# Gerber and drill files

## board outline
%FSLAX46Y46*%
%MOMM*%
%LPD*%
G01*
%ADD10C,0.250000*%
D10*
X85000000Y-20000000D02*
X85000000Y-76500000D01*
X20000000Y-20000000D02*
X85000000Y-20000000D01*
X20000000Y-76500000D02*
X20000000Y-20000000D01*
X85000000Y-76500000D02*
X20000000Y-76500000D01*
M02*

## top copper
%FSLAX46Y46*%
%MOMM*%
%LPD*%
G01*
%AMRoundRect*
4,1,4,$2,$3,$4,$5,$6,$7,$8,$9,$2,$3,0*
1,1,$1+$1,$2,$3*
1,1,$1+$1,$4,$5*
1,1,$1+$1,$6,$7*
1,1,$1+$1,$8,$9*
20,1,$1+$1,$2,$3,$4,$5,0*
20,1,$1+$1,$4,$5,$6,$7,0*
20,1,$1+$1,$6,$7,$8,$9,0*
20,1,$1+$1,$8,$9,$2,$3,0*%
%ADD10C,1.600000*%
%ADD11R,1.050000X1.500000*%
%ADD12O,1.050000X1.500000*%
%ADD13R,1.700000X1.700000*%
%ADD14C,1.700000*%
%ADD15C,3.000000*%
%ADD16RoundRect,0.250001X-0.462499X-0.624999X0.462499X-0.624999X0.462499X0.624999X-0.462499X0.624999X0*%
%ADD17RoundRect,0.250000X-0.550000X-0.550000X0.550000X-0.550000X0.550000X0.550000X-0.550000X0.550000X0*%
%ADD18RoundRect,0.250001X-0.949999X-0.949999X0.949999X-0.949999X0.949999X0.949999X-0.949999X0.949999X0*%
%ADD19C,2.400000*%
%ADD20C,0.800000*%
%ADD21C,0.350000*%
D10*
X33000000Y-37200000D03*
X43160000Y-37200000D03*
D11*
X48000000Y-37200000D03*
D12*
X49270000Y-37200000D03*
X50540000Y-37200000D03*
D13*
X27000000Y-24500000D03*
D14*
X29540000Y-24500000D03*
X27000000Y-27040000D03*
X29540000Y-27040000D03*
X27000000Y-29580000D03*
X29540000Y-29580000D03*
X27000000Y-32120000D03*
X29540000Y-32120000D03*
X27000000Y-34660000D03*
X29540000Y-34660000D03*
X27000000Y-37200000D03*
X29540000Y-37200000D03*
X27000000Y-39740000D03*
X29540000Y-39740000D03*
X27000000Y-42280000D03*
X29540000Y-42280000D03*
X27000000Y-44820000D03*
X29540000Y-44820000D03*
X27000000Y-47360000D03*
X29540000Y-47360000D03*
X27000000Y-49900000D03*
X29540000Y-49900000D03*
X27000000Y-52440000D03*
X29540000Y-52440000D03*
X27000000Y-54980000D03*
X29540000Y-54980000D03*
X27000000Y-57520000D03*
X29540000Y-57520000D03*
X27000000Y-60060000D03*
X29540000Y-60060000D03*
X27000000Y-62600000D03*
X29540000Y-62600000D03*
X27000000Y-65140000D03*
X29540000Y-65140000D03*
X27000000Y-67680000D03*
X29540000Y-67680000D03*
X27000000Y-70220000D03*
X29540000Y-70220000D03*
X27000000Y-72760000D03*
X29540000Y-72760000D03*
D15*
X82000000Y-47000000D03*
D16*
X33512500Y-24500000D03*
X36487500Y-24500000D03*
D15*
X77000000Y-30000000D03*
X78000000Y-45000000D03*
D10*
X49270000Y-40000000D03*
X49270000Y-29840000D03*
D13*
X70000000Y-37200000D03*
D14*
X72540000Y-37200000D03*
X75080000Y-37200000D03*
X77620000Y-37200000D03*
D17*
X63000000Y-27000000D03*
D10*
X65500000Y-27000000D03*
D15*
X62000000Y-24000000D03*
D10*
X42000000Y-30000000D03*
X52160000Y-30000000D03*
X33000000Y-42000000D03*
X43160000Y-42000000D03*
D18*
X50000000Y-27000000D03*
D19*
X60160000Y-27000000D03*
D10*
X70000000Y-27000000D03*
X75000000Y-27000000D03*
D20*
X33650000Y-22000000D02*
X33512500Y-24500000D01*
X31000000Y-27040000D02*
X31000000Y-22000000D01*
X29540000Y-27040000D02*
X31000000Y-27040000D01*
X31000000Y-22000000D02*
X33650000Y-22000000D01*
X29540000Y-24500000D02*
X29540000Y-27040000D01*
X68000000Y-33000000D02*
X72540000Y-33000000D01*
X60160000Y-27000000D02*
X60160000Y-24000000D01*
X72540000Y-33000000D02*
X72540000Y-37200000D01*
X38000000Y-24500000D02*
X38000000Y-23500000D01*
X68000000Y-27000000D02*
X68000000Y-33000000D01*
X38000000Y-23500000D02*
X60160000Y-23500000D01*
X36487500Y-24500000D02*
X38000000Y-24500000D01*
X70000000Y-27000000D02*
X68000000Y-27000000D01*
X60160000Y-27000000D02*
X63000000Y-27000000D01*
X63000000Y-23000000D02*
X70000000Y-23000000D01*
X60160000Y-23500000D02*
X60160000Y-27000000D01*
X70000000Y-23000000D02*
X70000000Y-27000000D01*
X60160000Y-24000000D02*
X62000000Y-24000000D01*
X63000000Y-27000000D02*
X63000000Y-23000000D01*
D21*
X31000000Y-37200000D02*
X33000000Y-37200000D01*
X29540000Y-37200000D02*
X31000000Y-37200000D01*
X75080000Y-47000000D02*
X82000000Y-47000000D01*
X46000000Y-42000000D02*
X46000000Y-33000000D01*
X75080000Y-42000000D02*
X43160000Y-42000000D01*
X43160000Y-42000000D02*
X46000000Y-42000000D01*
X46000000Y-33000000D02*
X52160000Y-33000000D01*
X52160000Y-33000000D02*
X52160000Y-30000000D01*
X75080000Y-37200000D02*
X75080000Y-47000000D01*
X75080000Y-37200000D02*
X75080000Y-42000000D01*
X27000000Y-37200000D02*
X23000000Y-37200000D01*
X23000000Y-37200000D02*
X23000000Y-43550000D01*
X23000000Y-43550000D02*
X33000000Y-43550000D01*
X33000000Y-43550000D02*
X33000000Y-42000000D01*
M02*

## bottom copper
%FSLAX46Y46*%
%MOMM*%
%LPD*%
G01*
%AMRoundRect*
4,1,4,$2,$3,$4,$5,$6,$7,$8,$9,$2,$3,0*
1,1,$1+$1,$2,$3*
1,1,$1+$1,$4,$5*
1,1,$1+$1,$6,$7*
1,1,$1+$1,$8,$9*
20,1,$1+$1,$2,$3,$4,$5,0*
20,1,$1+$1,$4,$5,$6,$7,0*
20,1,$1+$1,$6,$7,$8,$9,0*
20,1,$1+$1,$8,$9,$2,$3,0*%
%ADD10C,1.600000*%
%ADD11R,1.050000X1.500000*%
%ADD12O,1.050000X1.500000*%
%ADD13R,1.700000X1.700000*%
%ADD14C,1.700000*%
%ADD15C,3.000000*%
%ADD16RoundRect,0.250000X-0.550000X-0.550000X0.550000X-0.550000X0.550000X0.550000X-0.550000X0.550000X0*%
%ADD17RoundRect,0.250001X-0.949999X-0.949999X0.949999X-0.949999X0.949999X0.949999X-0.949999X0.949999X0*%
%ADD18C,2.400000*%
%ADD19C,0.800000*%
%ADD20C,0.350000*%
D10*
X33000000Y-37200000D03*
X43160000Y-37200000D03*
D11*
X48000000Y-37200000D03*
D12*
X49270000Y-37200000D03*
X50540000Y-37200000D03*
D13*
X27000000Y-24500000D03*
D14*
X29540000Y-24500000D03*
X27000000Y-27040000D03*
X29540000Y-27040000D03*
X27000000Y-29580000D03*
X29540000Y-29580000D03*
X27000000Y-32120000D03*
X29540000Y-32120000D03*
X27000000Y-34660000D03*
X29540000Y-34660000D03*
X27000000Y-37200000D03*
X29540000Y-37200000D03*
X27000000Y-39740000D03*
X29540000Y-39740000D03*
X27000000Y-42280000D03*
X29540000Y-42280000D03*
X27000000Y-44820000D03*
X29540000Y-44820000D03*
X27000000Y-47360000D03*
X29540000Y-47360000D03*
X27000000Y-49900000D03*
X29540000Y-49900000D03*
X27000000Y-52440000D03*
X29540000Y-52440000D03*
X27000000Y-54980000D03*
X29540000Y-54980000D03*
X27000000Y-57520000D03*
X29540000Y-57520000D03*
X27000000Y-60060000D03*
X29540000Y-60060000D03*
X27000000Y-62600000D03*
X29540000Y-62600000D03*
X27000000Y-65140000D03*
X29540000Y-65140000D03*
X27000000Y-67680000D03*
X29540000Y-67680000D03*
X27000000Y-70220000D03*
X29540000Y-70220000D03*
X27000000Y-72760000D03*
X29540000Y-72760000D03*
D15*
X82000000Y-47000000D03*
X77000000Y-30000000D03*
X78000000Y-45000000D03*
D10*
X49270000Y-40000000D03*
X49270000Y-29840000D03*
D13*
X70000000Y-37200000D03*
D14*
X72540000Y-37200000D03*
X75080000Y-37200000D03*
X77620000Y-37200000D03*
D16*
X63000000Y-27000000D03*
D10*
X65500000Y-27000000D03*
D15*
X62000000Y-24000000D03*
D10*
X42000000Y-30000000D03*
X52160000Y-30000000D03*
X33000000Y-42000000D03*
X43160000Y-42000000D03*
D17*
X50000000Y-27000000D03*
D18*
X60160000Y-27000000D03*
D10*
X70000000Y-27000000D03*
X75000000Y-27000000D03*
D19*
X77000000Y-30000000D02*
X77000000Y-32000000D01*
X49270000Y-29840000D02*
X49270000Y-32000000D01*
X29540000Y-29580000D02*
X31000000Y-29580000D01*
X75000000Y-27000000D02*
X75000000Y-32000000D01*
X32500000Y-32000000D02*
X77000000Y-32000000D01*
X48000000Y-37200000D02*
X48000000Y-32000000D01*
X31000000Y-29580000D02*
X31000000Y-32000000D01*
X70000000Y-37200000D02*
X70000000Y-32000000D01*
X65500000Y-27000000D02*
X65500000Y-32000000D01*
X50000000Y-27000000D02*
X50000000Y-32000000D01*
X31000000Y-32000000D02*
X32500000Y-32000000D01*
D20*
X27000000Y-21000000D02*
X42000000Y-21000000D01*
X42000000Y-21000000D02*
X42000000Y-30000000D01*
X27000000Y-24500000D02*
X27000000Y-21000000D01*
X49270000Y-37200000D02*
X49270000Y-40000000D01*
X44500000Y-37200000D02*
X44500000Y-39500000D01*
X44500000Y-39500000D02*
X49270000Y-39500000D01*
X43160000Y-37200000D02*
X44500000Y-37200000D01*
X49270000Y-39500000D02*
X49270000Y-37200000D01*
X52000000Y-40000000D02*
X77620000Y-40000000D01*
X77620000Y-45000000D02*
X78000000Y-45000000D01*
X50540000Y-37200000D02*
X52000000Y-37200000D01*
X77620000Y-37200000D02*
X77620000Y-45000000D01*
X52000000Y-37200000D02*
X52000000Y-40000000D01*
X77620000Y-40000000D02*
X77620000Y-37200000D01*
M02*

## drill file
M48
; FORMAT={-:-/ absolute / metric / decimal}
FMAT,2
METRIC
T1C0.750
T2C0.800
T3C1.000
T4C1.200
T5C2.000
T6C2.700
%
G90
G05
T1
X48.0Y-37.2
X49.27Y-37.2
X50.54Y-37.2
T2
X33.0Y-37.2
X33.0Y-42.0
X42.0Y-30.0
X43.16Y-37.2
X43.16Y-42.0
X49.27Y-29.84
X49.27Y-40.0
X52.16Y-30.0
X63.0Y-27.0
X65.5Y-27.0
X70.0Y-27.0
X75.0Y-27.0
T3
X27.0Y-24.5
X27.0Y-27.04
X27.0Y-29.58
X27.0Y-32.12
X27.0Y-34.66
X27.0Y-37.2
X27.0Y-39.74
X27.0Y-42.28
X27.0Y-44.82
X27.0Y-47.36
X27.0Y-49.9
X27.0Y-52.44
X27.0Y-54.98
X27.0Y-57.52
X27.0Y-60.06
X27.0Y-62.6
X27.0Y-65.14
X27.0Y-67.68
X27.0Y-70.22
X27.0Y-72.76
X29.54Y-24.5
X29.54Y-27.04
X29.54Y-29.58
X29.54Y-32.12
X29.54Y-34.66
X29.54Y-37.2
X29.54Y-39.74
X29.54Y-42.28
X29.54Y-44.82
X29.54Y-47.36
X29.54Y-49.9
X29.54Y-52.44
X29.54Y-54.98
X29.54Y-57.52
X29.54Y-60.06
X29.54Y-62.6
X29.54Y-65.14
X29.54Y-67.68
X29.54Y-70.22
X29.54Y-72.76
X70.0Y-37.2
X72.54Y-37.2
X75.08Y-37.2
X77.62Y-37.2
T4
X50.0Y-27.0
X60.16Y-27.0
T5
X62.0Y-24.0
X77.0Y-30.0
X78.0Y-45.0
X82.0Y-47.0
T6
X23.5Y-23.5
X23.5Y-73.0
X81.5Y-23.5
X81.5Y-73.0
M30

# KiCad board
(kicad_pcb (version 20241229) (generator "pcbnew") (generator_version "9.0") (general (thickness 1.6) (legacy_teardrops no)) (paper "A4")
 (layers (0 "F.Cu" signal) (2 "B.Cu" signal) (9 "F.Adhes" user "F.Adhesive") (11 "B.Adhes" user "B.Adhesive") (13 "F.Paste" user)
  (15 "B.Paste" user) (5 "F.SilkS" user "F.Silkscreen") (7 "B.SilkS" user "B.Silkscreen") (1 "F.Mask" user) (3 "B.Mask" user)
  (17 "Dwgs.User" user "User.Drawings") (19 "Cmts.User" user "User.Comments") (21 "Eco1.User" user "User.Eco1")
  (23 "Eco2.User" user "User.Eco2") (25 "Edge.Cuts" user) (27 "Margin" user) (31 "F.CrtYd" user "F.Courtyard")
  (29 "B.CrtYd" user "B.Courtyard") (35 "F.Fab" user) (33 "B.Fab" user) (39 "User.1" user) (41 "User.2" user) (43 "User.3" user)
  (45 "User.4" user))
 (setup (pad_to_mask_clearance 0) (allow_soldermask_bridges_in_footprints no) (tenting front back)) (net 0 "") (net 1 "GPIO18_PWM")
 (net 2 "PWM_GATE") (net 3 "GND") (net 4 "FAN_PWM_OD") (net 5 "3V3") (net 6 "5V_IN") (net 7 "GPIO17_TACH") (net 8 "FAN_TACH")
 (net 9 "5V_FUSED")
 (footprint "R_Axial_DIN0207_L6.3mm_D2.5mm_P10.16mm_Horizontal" (layer "F.Cu") (at 33 37.2)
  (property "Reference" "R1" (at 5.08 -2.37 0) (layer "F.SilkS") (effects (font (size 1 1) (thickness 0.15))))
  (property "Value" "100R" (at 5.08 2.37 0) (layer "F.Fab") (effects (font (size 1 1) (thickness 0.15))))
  (pad "1" thru_hole circle (at 0 0) (size 1.6 1.6) (drill 0.8) (layers "*.Cu" "*.Mask") (remove_unused_layers no) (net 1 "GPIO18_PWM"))
  (pad "2" thru_hole circle (at 10.16 0) (size 1.6 1.6) (drill 0.8) (layers "*.Cu" "*.Mask") (remove_unused_layers no) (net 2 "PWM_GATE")))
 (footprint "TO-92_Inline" (layer "F.Cu") (at 48 37.2)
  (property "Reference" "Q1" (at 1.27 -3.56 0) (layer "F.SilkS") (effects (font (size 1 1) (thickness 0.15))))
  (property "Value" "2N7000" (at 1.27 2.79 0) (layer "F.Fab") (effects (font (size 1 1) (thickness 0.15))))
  (pad "1" thru_hole rect (at 0 0) (size 1.05 1.5) (drill 0.75) (layers "*.Cu" "*.Mask") (remove_unused_layers no) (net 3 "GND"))
  (pad "2" thru_hole oval (at 1.27 0) (size 1.05 1.5) (drill 0.75) (layers "*.Cu" "*.Mask") (remove_unused_layers no) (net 2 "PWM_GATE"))
  (pad "3" thru_hole oval (at 2.54 0) (size 1.05 1.5) (drill 0.75) (layers "*.Cu" "*.Mask") (remove_unused_layers no) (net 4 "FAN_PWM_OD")))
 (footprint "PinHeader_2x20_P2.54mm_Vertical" (layer "F.Cu") (at 27 24.5)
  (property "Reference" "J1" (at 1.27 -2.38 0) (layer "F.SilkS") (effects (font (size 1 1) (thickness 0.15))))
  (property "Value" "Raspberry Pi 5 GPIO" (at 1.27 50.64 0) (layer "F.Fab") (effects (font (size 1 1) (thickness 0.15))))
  (pad "1" thru_hole rect (at 0 0) (size 1.7 1.7) (drill 1) (layers "*.Cu" "*.Mask") (remove_unused_layers no) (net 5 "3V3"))
  (pad "2" thru_hole circle (at 2.54 0) (size 1.7 1.7) (drill 1) (layers "*.Cu" "*.Mask") (remove_unused_layers no) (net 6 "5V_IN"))
  (pad "3" thru_hole circle (at 0 2.54) (size 1.7 1.7) (drill 1) (layers "*.Cu" "*.Mask") (remove_unused_layers no))
  (pad "4" thru_hole circle (at 2.54 2.54) (size 1.7 1.7) (drill 1) (layers "*.Cu" "*.Mask") (remove_unused_layers no) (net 6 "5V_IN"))
  (pad "5" thru_hole circle (at 0 5.08) (size 1.7 1.7) (drill 1) (layers "*.Cu" "*.Mask") (remove_unused_layers no))
  (pad "6" thru_hole circle (at 2.54 5.08) (size 1.7 1.7) (drill 1) (layers "*.Cu" "*.Mask") (remove_unused_layers no) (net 3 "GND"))
  (pad "7" thru_hole circle (at 0 7.62) (size 1.7 1.7) (drill 1) (layers "*.Cu" "*.Mask") (remove_unused_layers no))
  (pad "8" thru_hole circle (at 2.54 7.62) (size 1.7 1.7) (drill 1) (layers "*.Cu" "*.Mask") (remove_unused_layers no))
  (pad "9" thru_hole circle (at 0 10.16) (size 1.7 1.7) (drill 1) (layers "*.Cu" "*.Mask") (remove_unused_layers no))
  (pad "10" thru_hole circle (at 2.54 10.16) (size 1.7 1.7) (drill 1) (layers "*.Cu" "*.Mask") (remove_unused_layers no))
  (pad "11" thru_hole circle (at 0 12.7) (size 1.7 1.7) (drill 1) (layers "*.Cu" "*.Mask") (remove_unused_layers no) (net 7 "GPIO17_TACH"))
  (pad "12" thru_hole circle (at 2.54 12.7) (size 1.7 1.7) (drill 1) (layers "*.Cu" "*.Mask") (remove_unused_layers no) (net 1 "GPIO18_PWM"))
  (pad "13" thru_hole circle (at 0 15.24) (size 1.7 1.7) (drill 1) (layers "*.Cu" "*.Mask") (remove_unused_layers no))
  (pad "14" thru_hole circle (at 2.54 15.24) (size 1.7 1.7) (drill 1) (layers "*.Cu" "*.Mask") (remove_unused_layers no))
  (pad "15" thru_hole circle (at 0 17.78) (size 1.7 1.7) (drill 1) (layers "*.Cu" "*.Mask") (remove_unused_layers no))
  (pad "16" thru_hole circle (at 2.54 17.78) (size 1.7 1.7) (drill 1) (layers "*.Cu" "*.Mask") (remove_unused_layers no))
  (pad "17" thru_hole circle (at 0 20.32) (size 1.7 1.7) (drill 1) (layers "*.Cu" "*.Mask") (remove_unused_layers no))
  (pad "18" thru_hole circle (at 2.54 20.32) (size 1.7 1.7) (drill 1) (layers "*.Cu" "*.Mask") (remove_unused_layers no))
  (pad "19" thru_hole circle (at 0 22.86) (size 1.7 1.7) (drill 1) (layers "*.Cu" "*.Mask") (remove_unused_layers no))
  (pad "20" thru_hole circle (at 2.54 22.86) (size 1.7 1.7) (drill 1) (layers "*.Cu" "*.Mask") (remove_unused_layers no))
  (pad "21" thru_hole circle (at 0 25.4) (size 1.7 1.7) (drill 1) (layers "*.Cu" "*.Mask") (remove_unused_layers no))
  (pad "22" thru_hole circle (at 2.54 25.4) (size 1.7 1.7) (drill 1) (layers "*.Cu" "*.Mask") (remove_unused_layers no))
  (pad "23" thru_hole circle (at 0 27.94) (size 1.7 1.7) (drill 1) (layers "*.Cu" "*.Mask") (remove_unused_layers no))
  (pad "24" thru_hole circle (at 2.54 27.94) (size 1.7 1.7) (drill 1) (layers "*.Cu" "*.Mask") (remove_unused_layers no))
  (pad "25" thru_hole circle (at 0 30.48) (size 1.7 1.7) (drill 1) (layers "*.Cu" "*.Mask") (remove_unused_layers no))
  (pad "26" thru_hole circle (at 2.54 30.48) (size 1.7 1.7) (drill 1) (layers "*.Cu" "*.Mask") (remove_unused_layers no))
  (pad "27" thru_hole circle (at 0 33.02) (size 1.7 1.7) (drill 1) (layers "*.Cu" "*.Mask") (remove_unused_layers no))
  (pad "28" thru_hole circle (at 2.54 33.02) (size 1.7 1.7) (drill 1) (layers "*.Cu" "*.Mask") (remove_unused_layers no))
  (pad "29" thru_hole circle (at 0 35.56) (size 1.7 1.7) (drill 1) (layers "*.Cu" "*.Mask") (remove_unused_layers no))
  (pad "30" thru_hole circle (at 2.54 35.56) (size 1.7 1.7) (drill 1) (layers "*.Cu" "*.Mask") (remove_unused_layers no))
  (pad "31" thru_hole circle (at 0 38.1) (size 1.7 1.7) (drill 1) (layers "*.Cu" "*.Mask") (remove_unused_layers no))
  (pad "32" thru_hole circle (at 2.54 38.1) (size 1.7 1.7) (drill 1) (layers "*.Cu" "*.Mask") (remove_unused_layers no))
  (pad "33" thru_hole circle (at 0 40.64) (size 1.7 1.7) (drill 1) (layers "*.Cu" "*.Mask") (remove_unused_layers no))
  (pad "34" thru_hole circle (at 2.54 40.64) (size 1.7 1.7) (drill 1) (layers "*.Cu" "*.Mask") (remove_unused_layers no))
  (pad "35" thru_hole circle (at 0 43.18) (size 1.7 1.7) (drill 1) (layers "*.Cu" "*.Mask") (remove_unused_layers no))
  (pad "36" thru_hole circle (at 2.54 43.18) (size 1.7 1.7) (drill 1) (layers "*.Cu" "*.Mask") (remove_unused_layers no))
  (pad "37" thru_hole circle (at 0 45.72) (size 1.7 1.7) (drill 1) (layers "*.Cu" "*.Mask") (remove_unused_layers no))
  (pad "38" thru_hole circle (at 2.54 45.72) (size 1.7 1.7) (drill 1) (layers "*.Cu" "*.Mask") (remove_unused_layers no))
  (pad "39" thru_hole circle (at 0 48.26) (size 1.7 1.7) (drill 1) (layers "*.Cu" "*.Mask") (remove_unused_layers no))
  (pad "40" thru_hole circle (at 2.54 48.26) (size 1.7 1.7) (drill 1) (layers "*.Cu" "*.Mask") (remove_unused_layers no)))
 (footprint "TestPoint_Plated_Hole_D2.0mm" (layer "F.Cu") (at 82 47)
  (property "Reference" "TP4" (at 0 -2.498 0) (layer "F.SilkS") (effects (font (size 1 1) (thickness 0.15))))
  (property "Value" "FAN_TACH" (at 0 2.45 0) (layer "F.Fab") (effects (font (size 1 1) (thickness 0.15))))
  (pad "1" thru_hole circle (at 0 0) (size 3 3) (drill 2) (layers "*.Cu" "*.Mask") (remove_unused_layers no) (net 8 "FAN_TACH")))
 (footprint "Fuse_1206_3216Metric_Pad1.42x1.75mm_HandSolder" (layer "F.Cu") (at 35 24.5)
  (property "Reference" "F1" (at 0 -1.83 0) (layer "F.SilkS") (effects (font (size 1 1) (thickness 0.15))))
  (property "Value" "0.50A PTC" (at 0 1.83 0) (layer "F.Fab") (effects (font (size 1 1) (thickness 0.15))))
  (pad "1" smd roundrect (at -1.4875 0) (size 1.425 1.75) (layers "F.Cu" "F.Mask" "F.Paste") (roundrect_rratio 0.175439) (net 6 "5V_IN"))
  (pad "2" smd roundrect (at 1.4875 0) (size 1.425 1.75) (layers "F.Cu" "F.Mask" "F.Paste") (roundrect_rratio 0.175439) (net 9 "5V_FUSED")))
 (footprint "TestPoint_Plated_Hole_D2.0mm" (layer "F.Cu") (at 77 30)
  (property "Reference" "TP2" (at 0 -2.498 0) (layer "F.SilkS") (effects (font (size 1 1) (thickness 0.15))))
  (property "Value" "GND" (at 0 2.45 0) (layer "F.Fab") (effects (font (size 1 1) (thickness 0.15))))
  (pad "1" thru_hole circle (at 0 0) (size 3 3) (drill 2) (layers "*.Cu" "*.Mask") (remove_unused_layers no) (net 3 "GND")))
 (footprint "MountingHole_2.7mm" (layer "F.Cu") (at 81.5 23.5)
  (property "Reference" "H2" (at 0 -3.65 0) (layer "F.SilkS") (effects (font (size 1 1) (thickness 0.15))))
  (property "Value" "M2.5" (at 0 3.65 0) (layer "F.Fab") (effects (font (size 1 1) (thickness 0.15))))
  (pad "" np_thru_hole circle (at 0 0) (size 2.7 2.7) (drill 2.7) (layers "*.Cu" "*.Mask")))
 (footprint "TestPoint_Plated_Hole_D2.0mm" (layer "F.Cu") (at 78 45)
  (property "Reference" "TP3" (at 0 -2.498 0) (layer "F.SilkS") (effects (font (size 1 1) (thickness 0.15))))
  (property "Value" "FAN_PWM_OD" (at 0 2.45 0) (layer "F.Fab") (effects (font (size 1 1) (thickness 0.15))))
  (pad "1" thru_hole circle (at 0 0) (size 3 3) (drill 2) (layers "*.Cu" "*.Mask") (remove_unused_layers no) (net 4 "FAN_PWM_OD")))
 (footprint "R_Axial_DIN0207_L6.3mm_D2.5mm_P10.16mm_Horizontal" (layer "F.Cu") (at 49.27 40 90)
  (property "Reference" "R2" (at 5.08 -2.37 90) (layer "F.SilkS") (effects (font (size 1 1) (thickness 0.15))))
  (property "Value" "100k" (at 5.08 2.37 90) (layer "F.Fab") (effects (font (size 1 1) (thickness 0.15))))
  (pad "1" thru_hole circle (at 0 0 90) (size 1.6 1.6) (drill 0.8) (layers "*.Cu" "*.Mask") (remove_unused_layers no) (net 2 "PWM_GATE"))
  (pad "2" thru_hole circle (at 10.16 0 90) (size 1.6 1.6) (drill 0.8) (layers "*.Cu" "*.Mask") (remove_unused_layers no) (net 3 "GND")))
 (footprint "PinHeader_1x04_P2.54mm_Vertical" (layer "F.Cu") (at 70 37.2 90)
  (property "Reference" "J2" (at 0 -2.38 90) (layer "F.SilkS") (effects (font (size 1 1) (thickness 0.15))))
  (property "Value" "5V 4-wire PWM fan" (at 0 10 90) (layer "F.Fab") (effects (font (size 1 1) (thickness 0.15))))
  (pad "1" thru_hole rect (at 0 0 90) (size 1.7 1.7) (drill 1) (layers "*.Cu" "*.Mask") (remove_unused_layers no) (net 3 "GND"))
  (pad "2" thru_hole circle (at 0 2.54 90) (size 1.7 1.7) (drill 1) (layers "*.Cu" "*.Mask") (remove_unused_layers no) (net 9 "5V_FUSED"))
  (pad "3" thru_hole circle (at 0 5.08 90) (size 1.7 1.7) (drill 1) (layers "*.Cu" "*.Mask") (remove_unused_layers no) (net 8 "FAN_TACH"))
  (pad "4" thru_hole circle (at 0 7.62 90) (size 1.7 1.7) (drill 1) (layers "*.Cu" "*.Mask") (remove_unused_layers no) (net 4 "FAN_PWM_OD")))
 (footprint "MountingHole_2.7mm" (layer "F.Cu") (at 81.5 73)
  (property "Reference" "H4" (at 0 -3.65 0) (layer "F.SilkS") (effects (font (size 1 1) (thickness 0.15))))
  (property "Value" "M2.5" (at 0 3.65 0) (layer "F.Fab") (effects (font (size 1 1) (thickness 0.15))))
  (pad "" np_thru_hole circle (at 0 0) (size 2.7 2.7) (drill 2.7) (layers "*.Cu" "*.Mask")))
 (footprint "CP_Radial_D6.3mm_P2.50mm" (layer "F.Cu") (at 63 27)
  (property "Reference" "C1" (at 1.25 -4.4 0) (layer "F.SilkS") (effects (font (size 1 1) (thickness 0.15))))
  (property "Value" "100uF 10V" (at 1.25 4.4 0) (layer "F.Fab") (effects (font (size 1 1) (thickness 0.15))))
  (pad "1" thru_hole roundrect (at 0 0) (size 1.6 1.6) (drill 0.8) (layers "*.Cu" "*.Mask") (remove_unused_layers no)
   (roundrect_rratio 0.15625) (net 9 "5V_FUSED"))
  (pad "2" thru_hole circle (at 2.5 0) (size 1.6 1.6) (drill 0.8) (layers "*.Cu" "*.Mask") (remove_unused_layers no) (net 3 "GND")))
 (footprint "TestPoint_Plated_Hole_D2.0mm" (layer "F.Cu") (at 62 24)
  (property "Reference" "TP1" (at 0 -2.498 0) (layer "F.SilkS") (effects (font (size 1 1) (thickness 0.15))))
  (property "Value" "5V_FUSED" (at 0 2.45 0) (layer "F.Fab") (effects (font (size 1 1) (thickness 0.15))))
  (pad "1" thru_hole circle (at 0 0) (size 3 3) (drill 2) (layers "*.Cu" "*.Mask") (remove_unused_layers no) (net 9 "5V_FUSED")))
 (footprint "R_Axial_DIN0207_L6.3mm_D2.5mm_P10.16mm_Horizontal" (layer "F.Cu") (at 42 30)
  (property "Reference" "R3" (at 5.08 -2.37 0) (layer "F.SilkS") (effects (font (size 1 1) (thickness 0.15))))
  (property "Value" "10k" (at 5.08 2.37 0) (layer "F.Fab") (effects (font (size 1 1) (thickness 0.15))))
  (pad "1" thru_hole circle (at 0 0) (size 1.6 1.6) (drill 0.8) (layers "*.Cu" "*.Mask") (remove_unused_layers no) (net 5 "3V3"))
  (pad "2" thru_hole circle (at 10.16 0) (size 1.6 1.6) (drill 0.8) (layers "*.Cu" "*.Mask") (remove_unused_layers no) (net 8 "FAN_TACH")))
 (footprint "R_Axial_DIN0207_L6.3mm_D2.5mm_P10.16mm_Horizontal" (layer "F.Cu") (at 33 42)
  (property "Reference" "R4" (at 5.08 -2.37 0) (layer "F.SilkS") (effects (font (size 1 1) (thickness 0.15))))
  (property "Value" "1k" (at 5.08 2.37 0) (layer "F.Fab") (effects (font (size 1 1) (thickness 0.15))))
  (pad "1" thru_hole circle (at 0 0) (size 1.6 1.6) (drill 0.8) (layers "*.Cu" "*.Mask") (remove_unused_layers no) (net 7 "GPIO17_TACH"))
  (pad "2" thru_hole circle (at 10.16 0) (size 1.6 1.6) (drill 0.8) (layers "*.Cu" "*.Mask") (remove_unused_layers no) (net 8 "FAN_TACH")))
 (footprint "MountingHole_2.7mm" (layer "F.Cu") (at 23.5 73)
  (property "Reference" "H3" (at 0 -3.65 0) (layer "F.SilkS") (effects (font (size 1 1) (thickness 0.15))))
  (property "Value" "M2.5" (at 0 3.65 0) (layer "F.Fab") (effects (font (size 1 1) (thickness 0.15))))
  (pad "" np_thru_hole circle (at 0 0) (size 2.7 2.7) (drill 2.7) (layers "*.Cu" "*.Mask")))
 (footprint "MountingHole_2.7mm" (layer "F.Cu") (at 23.5 23.5)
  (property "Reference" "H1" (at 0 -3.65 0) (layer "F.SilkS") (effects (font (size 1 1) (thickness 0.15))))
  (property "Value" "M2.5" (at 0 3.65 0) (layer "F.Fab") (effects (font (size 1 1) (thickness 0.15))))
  (pad "" np_thru_hole circle (at 0 0) (size 2.7 2.7) (drill 2.7) (layers "*.Cu" "*.Mask")))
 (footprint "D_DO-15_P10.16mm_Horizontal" (layer "F.Cu") (at 50 27)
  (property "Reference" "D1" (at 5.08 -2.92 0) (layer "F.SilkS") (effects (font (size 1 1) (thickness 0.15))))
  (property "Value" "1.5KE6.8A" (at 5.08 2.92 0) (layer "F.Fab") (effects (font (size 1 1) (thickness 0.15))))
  (pad "1" thru_hole roundrect (at 0 0) (size 2.4 2.4) (drill 1.2) (layers "*.Cu" "*.Mask") (remove_unused_layers no)
   (roundrect_rratio 0.104167) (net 3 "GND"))
  (pad "2" thru_hole circle (at 10.16 0) (size 2.4 2.4) (drill 1.2) (layers "*.Cu" "*.Mask") (remove_unused_layers no) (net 9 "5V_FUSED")))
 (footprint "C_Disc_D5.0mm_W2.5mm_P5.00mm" (layer "F.Cu") (at 70 27)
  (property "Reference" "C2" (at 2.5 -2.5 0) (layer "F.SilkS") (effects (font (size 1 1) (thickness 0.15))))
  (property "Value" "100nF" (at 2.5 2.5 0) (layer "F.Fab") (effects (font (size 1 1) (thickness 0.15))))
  (pad "1" thru_hole circle (at 0 0) (size 1.6 1.6) (drill 0.8) (layers "*.Cu" "*.Mask") (remove_unused_layers no) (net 9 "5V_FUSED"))
  (pad "2" thru_hole circle (at 5 0) (size 1.6 1.6) (drill 0.8) (layers "*.Cu" "*.Mask") (remove_unused_layers no) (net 3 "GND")))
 (gr_line (start 85 20) (end 85 76.5) (stroke (width 0.25) (type default)) (layer "Edge.Cuts"))
 (gr_line (start 20 20) (end 85 20) (stroke (width 0.25) (type default)) (layer "Edge.Cuts"))
 (gr_line (start 20 76.5) (end 20 20) (stroke (width 0.25) (type default)) (layer "Edge.Cuts"))
 (gr_line (start 85 76.5) (end 20 76.5) (stroke (width 0.25) (type default)) (layer "Edge.Cuts"))
 (segment (start 77 30) (end 77 32) (width 0.8) (layer "B.Cu") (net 3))
 (segment (start 49.27 29.84) (end 49.27 32) (width 0.8) (layer "B.Cu") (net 3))
 (segment (start 29.54 29.58) (end 31 29.58) (width 0.8) (layer "B.Cu") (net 3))
 (segment (start 75 27) (end 75 32) (width 0.8) (layer "B.Cu") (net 3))
 (segment (start 32.5 32) (end 77 32) (width 0.8) (layer "B.Cu") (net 3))
 (segment (start 48 37.2) (end 48 32) (width 0.8) (layer "B.Cu") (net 3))
 (segment (start 31 29.58) (end 31 32) (width 0.8) (layer "B.Cu") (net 3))
 (segment (start 70 37.2) (end 70 32) (width 0.8) (layer "B.Cu") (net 3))
 (segment (start 65.5 27) (end 65.5 32) (width 0.8) (layer "B.Cu") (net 3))
 (segment (start 50 27) (end 50 32) (width 0.8) (layer "B.Cu") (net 3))
 (segment (start 31 32) (end 32.5 32) (width 0.8) (layer "B.Cu") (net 3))
 (segment (start 33.65 22) (end 33.5125 24.5) (width 0.8) (layer "F.Cu") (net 6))
 (segment (start 31 27.04) (end 31 22) (width 0.8) (layer "F.Cu") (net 6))
 (segment (start 29.54 27.04) (end 31 27.04) (width 0.8) (layer "F.Cu") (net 6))
 (segment (start 31 22) (end 33.65 22) (width 0.8) (layer "F.Cu") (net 6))
 (segment (start 29.54 24.5) (end 29.54 27.04) (width 0.8) (layer "F.Cu") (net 6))
 (segment (start 68 33) (end 72.54 33) (width 0.8) (layer "F.Cu") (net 9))
 (segment (start 60.16 27) (end 60.16 24) (width 0.8) (layer "F.Cu") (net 9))
 (segment (start 72.54 33) (end 72.54 37.2) (width 0.8) (layer "F.Cu") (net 9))
 (segment (start 38 24.5) (end 38 23.5) (width 0.8) (layer "F.Cu") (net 9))
 (segment (start 68 27) (end 68 33) (width 0.8) (layer "F.Cu") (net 9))
 (segment (start 38 23.5) (end 60.16 23.5) (width 0.8) (layer "F.Cu") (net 9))
 (segment (start 36.4875 24.5) (end 38 24.5) (width 0.8) (layer "F.Cu") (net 9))
 (segment (start 70 27) (end 68 27) (width 0.8) (layer "F.Cu") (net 9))
 (segment (start 60.16 27) (end 63 27) (width 0.8) (layer "F.Cu") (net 9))
 (segment (start 63 23) (end 70 23) (width 0.8) (layer "F.Cu") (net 9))
 (segment (start 60.16 23.5) (end 60.16 27) (width 0.8) (layer "F.Cu") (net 9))
 (segment (start 70 23) (end 70 27) (width 0.8) (layer "F.Cu") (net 9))
 (segment (start 60.16 24) (end 62 24) (width 0.8) (layer "F.Cu") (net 9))
 (segment (start 63 27) (end 63 23) (width 0.8) (layer "F.Cu") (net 9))
 (segment (start 27 21) (end 42 21) (width 0.35) (layer "B.Cu") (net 5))
 (segment (start 42 21) (end 42 30) (width 0.35) (layer "B.Cu") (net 5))
 (segment (start 27 24.5) (end 27 21) (width 0.35) (layer "B.Cu") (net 5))
 (segment (start 31 37.2) (end 33 37.2) (width 0.35) (layer "F.Cu") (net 1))
 (segment (start 29.54 37.2) (end 31 37.2) (width 0.35) (layer "F.Cu") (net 1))
 (segment (start 49.27 37.2) (end 49.27 40) (width 0.35) (layer "B.Cu") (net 2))
 (segment (start 44.5 37.2) (end 44.5 39.5) (width 0.35) (layer "B.Cu") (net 2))
 (segment (start 44.5 39.5) (end 49.27 39.5) (width 0.35) (layer "B.Cu") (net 2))
 (segment (start 43.16 37.2) (end 44.5 37.2) (width 0.35) (layer "B.Cu") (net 2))
 (segment (start 49.27 39.5) (end 49.27 37.2) (width 0.35) (layer "B.Cu") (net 2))
 (segment (start 52 40) (end 77.62 40) (width 0.35) (layer "B.Cu") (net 4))
 (segment (start 77.62 45) (end 78 45) (width 0.35) (layer "B.Cu") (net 4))
 (segment (start 50.54 37.2) (end 52 37.2) (width 0.35) (layer "B.Cu") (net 4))
 (segment (start 77.62 37.2) (end 77.62 45) (width 0.35) (layer "B.Cu") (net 4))
 (segment (start 52 37.2) (end 52 40) (width 0.35) (layer "B.Cu") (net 4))
 (segment (start 77.62 40) (end 77.62 37.2) (width 0.35) (layer "B.Cu") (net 4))
 (segment (start 75.08 47) (end 82 47) (width 0.35) (layer "F.Cu") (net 8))
 (segment (start 46 42) (end 46 33) (width 0.35) (layer "F.Cu") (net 8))
 (segment (start 75.08 42) (end 43.16 42) (width 0.35) (layer "F.Cu") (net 8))
 (segment (start 43.16 42) (end 46 42) (width 0.35) (layer "F.Cu") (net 8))
 (segment (start 46 33) (end 52.16 33) (width 0.35) (layer "F.Cu") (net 8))
 (segment (start 52.16 33) (end 52.16 30) (width 0.35) (layer "F.Cu") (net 8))
 (segment (start 75.08 37.2) (end 75.08 47) (width 0.35) (layer "F.Cu") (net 8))
 (segment (start 75.08 37.2) (end 75.08 42) (width 0.35) (layer "F.Cu") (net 8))
 (segment (start 27 37.2) (end 23 37.2) (width 0.35) (layer "F.Cu") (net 7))
 (segment (start 23 37.2) (end 23 43.55) (width 0.35) (layer "F.Cu") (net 7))
 (segment (start 23 43.55) (end 33 43.55) (width 0.35) (layer "F.Cu") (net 7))
 (segment (start 33 43.55) (end 33 42) (width 0.35) (layer "F.Cu") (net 7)))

